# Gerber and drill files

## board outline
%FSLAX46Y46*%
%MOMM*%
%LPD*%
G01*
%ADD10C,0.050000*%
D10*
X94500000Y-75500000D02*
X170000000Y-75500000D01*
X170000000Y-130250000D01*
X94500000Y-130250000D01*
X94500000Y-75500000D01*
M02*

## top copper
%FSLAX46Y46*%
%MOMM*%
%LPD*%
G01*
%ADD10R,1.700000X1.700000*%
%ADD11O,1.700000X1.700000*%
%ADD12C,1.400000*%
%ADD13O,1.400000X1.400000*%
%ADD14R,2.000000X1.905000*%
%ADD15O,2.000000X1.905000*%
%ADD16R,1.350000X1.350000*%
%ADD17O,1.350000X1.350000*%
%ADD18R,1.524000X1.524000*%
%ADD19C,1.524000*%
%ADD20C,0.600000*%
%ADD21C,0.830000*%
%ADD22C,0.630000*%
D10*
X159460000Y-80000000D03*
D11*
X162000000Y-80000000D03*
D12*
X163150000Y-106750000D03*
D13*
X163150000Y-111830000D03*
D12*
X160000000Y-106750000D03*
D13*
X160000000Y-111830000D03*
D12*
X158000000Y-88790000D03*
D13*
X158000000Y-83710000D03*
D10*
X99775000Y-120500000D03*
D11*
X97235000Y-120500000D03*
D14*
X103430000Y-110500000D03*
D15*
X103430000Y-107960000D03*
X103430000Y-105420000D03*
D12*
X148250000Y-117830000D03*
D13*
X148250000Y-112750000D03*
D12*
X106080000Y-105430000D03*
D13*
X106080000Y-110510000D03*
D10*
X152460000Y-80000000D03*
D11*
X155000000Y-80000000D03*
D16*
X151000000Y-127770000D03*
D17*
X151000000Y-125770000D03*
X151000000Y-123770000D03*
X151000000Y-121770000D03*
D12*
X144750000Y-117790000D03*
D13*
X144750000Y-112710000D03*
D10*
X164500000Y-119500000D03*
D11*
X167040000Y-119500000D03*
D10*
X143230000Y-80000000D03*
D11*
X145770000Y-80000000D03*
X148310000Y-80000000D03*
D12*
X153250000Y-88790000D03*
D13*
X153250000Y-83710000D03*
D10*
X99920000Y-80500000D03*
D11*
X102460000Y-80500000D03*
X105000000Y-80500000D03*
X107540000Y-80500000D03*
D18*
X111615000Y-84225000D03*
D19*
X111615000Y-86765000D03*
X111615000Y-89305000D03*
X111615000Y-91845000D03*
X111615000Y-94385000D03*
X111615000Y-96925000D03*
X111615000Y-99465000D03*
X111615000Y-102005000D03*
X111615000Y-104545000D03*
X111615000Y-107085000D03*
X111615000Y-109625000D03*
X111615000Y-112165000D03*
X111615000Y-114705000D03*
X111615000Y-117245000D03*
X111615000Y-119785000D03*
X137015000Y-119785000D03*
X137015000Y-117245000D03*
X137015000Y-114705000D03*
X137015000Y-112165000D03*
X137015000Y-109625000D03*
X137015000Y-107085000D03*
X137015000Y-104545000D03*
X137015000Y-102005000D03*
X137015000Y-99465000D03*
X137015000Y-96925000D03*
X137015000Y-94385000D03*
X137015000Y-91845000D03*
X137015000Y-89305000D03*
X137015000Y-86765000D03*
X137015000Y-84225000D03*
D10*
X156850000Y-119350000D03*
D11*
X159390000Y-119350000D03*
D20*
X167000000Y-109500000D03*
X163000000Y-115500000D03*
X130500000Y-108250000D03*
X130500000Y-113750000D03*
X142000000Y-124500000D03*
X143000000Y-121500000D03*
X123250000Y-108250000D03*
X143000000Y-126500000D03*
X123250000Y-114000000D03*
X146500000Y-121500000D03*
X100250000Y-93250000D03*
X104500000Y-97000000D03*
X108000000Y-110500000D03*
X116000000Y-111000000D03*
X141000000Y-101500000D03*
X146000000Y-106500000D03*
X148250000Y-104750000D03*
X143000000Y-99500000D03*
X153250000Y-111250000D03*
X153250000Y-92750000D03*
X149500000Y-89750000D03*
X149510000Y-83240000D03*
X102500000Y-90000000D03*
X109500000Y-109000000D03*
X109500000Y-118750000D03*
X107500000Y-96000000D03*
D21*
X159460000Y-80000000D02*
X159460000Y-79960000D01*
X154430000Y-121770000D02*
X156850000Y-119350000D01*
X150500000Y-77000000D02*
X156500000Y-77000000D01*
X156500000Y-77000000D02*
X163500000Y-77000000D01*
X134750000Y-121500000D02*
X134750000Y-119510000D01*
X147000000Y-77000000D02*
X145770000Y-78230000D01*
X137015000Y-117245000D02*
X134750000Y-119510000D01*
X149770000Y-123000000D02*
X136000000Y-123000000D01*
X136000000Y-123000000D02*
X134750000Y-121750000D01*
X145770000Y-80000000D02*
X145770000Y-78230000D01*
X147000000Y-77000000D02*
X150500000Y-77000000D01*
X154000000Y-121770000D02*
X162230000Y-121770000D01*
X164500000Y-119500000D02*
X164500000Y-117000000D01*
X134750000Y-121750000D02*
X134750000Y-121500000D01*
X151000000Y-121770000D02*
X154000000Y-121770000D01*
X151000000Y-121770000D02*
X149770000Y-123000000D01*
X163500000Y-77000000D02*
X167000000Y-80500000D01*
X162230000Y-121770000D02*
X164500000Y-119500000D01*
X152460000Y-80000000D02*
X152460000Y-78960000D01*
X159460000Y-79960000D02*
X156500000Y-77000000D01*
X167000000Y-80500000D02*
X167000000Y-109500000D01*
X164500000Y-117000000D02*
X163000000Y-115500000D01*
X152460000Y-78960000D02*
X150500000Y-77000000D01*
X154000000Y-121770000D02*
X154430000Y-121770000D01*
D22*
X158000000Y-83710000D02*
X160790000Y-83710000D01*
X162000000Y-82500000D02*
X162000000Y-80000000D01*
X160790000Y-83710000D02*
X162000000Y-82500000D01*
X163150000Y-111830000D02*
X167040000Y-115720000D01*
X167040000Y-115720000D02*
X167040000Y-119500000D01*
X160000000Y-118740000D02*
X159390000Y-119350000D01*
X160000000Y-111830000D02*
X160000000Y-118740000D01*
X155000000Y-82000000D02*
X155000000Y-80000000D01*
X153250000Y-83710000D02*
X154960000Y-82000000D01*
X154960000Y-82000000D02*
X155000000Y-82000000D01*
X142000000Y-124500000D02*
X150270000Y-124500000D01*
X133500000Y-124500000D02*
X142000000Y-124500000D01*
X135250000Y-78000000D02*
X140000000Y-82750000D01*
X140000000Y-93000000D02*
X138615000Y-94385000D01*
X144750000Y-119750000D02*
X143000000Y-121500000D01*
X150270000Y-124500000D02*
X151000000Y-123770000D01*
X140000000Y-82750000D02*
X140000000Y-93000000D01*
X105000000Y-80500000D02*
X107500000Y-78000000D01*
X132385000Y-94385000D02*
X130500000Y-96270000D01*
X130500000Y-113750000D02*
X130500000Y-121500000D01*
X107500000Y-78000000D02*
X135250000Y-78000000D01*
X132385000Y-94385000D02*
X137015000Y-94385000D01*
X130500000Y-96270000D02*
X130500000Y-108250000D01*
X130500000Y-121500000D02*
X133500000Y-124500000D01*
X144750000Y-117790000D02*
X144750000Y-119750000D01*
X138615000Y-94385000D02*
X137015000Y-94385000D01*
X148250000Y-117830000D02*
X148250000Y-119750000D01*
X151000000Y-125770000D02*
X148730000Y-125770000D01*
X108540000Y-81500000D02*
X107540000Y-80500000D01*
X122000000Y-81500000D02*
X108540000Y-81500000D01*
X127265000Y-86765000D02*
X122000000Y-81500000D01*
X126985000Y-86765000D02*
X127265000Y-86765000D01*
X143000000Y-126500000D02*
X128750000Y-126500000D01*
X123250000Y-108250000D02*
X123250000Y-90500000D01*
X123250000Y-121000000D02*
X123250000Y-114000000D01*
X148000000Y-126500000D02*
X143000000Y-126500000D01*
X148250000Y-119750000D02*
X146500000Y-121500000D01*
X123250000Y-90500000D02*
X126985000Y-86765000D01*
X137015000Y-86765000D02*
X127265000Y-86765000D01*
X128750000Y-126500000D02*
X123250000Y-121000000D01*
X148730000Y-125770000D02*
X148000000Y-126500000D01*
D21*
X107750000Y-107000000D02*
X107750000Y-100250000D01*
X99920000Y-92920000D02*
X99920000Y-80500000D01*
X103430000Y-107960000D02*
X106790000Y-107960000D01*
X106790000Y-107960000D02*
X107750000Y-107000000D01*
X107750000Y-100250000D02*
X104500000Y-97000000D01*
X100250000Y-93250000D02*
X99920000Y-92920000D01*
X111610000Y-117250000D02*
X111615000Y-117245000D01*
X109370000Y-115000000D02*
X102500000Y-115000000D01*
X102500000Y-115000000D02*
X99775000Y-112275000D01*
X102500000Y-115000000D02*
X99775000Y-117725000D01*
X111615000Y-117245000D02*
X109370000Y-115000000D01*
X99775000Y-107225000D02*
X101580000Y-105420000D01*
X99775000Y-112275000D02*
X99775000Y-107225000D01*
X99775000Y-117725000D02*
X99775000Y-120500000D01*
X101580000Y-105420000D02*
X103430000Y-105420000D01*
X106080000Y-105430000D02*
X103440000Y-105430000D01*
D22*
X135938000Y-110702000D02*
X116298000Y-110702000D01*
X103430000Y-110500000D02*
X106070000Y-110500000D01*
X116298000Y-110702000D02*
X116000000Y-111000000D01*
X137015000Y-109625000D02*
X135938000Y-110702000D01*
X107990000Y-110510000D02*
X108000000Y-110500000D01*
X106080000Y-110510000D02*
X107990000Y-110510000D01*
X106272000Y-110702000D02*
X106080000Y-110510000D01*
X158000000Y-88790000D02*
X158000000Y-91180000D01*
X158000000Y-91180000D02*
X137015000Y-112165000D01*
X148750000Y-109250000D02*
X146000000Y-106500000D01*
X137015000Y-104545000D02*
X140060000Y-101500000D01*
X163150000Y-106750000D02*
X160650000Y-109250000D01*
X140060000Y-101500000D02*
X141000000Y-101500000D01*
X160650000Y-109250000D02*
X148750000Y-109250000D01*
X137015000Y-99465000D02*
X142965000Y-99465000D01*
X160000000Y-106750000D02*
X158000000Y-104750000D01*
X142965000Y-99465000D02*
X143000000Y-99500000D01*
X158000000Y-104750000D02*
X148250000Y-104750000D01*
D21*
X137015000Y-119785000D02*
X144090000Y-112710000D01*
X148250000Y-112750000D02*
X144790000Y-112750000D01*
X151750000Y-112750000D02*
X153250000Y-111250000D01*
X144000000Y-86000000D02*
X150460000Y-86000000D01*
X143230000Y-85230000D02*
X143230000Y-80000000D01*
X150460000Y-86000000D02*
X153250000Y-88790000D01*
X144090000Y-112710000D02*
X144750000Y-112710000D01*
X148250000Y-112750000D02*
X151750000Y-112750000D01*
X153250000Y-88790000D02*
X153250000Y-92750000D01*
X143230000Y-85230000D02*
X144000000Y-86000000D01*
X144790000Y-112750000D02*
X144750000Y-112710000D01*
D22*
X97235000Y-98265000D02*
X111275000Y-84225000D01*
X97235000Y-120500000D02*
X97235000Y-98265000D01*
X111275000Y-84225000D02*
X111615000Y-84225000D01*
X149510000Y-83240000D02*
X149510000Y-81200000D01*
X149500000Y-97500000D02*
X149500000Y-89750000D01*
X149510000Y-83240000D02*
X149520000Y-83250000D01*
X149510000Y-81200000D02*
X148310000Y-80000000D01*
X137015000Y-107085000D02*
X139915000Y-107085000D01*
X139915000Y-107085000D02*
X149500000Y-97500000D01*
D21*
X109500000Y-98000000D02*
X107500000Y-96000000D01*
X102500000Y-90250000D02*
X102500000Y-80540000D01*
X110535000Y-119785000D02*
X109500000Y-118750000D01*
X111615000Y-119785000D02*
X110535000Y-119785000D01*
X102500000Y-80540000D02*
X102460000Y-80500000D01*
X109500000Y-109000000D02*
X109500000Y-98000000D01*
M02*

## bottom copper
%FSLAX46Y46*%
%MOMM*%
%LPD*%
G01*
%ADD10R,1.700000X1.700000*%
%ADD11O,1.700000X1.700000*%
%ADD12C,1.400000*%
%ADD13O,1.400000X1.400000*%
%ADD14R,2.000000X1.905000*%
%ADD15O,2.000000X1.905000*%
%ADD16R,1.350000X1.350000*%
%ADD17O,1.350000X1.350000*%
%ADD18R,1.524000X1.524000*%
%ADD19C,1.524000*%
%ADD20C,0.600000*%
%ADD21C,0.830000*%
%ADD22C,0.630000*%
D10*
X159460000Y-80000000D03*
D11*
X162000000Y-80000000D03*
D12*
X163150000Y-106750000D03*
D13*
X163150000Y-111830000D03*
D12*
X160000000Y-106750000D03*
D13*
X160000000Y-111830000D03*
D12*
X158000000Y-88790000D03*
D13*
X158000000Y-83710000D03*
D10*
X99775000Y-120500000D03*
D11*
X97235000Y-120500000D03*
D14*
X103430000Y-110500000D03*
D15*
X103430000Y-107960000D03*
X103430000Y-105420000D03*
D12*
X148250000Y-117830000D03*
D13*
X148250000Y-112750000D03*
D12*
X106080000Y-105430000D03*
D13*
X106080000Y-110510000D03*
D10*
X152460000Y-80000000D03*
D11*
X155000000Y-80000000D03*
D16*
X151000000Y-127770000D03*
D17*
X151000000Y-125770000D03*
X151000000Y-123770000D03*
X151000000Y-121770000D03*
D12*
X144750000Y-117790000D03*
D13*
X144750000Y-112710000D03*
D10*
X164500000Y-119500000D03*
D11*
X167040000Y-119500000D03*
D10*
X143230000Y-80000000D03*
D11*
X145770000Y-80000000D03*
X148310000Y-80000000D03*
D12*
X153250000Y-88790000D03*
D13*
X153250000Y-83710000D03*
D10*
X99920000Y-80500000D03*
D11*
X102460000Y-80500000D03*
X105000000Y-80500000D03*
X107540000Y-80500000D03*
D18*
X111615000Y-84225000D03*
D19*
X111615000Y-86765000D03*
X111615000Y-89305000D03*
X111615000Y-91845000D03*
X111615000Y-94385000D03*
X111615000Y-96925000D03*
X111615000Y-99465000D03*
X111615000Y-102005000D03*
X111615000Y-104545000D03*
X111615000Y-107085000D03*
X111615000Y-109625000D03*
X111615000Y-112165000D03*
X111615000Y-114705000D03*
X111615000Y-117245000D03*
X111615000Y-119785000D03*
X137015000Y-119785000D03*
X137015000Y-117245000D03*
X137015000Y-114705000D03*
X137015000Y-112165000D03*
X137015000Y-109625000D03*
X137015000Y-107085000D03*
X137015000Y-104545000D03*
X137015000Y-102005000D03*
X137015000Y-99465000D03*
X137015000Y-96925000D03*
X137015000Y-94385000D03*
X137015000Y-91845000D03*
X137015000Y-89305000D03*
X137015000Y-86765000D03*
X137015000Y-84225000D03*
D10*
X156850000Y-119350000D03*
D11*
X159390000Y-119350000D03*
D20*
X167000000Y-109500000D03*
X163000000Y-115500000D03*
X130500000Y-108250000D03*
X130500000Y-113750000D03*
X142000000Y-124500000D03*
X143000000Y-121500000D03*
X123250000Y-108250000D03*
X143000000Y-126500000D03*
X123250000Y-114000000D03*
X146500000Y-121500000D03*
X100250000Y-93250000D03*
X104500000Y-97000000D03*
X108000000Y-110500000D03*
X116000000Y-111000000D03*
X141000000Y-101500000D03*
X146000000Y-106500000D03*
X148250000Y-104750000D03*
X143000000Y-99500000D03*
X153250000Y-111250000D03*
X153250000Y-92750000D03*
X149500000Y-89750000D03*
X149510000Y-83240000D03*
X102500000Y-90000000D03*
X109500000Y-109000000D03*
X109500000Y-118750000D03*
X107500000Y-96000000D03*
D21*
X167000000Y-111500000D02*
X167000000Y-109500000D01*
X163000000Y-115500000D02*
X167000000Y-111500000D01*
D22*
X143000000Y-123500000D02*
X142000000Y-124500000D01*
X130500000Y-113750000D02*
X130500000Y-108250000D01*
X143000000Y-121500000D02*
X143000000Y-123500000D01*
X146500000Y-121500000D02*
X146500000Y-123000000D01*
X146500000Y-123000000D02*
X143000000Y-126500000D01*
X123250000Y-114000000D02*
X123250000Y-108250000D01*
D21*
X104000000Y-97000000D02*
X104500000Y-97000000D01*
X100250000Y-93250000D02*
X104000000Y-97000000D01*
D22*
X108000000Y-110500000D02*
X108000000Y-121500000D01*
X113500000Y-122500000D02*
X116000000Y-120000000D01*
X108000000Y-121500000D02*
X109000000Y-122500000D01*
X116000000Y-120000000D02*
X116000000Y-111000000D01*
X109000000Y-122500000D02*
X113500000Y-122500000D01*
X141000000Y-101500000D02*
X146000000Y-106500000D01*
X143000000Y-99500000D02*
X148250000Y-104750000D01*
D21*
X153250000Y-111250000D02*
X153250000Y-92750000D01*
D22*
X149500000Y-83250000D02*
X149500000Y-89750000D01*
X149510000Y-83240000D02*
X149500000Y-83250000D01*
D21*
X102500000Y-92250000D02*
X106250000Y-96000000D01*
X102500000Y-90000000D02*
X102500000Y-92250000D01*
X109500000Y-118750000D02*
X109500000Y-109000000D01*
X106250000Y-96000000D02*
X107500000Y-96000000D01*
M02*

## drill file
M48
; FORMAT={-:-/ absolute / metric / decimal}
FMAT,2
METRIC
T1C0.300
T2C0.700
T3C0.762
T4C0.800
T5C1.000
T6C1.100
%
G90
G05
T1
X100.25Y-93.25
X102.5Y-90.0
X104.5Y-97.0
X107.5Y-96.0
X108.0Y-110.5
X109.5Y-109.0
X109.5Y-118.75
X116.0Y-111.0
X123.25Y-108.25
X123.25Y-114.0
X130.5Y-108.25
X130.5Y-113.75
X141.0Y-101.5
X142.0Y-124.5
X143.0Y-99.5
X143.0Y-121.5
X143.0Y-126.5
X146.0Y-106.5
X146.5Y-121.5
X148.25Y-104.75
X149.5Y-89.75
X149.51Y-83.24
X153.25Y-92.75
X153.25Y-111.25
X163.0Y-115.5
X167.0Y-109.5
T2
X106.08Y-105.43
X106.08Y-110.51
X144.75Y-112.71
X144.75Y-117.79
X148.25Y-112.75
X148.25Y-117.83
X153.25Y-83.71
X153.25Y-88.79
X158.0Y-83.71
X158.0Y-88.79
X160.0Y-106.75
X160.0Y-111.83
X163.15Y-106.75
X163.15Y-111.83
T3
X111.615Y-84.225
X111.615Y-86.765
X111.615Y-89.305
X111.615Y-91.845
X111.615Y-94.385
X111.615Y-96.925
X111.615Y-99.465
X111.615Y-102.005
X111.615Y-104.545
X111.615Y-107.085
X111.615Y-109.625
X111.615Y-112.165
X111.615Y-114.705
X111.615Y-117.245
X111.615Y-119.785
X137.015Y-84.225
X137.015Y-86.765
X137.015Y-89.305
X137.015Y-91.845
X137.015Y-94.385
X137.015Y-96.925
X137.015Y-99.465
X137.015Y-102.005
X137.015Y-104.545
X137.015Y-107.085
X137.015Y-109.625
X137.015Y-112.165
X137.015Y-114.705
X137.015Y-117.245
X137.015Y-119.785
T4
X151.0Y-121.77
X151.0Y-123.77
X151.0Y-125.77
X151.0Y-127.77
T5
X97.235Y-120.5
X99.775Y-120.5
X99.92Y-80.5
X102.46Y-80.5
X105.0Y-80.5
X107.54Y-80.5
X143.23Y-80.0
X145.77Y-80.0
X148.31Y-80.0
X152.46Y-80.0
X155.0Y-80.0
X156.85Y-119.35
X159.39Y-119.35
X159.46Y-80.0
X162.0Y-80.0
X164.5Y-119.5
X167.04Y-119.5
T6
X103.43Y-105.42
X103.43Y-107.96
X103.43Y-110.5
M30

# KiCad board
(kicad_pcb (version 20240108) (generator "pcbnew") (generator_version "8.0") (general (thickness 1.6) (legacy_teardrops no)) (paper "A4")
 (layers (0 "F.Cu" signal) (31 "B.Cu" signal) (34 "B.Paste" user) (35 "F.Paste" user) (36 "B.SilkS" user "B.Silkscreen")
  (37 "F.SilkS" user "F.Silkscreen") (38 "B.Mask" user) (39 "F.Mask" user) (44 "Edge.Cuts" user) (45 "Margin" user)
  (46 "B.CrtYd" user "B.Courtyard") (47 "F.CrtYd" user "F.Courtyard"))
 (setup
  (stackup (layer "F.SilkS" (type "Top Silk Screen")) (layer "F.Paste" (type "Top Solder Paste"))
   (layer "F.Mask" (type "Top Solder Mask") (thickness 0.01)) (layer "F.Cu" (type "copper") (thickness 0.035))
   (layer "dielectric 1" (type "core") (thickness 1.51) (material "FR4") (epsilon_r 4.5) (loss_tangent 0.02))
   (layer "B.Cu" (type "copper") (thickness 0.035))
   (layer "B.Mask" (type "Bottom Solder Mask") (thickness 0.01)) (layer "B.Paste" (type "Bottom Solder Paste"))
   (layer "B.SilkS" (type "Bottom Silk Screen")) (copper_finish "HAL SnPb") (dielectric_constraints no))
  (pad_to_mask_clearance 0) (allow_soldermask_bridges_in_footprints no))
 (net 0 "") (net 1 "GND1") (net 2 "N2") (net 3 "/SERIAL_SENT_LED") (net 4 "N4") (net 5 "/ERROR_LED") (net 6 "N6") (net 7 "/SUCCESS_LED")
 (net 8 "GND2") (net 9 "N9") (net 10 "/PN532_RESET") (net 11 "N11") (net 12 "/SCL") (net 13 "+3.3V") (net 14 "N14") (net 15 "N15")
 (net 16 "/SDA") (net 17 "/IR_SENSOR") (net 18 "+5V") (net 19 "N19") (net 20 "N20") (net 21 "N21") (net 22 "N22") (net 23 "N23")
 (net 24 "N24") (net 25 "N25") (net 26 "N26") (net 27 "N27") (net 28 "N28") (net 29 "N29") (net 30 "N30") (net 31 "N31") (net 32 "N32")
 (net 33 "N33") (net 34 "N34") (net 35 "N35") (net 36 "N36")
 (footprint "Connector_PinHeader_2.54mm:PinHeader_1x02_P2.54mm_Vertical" (layer "F.Cu") (at 159.46 80 90)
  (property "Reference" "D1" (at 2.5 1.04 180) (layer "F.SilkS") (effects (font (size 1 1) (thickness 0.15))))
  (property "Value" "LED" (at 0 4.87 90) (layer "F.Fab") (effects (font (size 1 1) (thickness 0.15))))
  (pad "1" thru_hole rect (at 0 0 90) (size 1.7 1.7) (drill 1) (layers "*.Cu" "*.Mask") (remove_unused_layers no) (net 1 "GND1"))
  (pad "2" thru_hole oval (at 0 2.54 90) (size 1.7 1.7) (drill 1) (layers "*.Cu" "*.Mask") (remove_unused_layers no) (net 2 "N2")))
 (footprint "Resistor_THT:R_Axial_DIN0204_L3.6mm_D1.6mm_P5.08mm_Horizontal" (layer "F.Cu") (at 163.15 106.75 -90)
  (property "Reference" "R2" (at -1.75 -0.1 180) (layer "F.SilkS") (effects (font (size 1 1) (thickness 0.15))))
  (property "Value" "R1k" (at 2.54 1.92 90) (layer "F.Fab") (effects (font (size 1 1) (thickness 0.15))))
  (pad "1" thru_hole circle (at 0 0 270) (size 1.4 1.4) (drill 0.7) (layers "*.Cu" "*.Mask") (remove_unused_layers no)
   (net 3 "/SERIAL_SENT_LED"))
  (pad "2" thru_hole oval (at 5.08 0 270) (size 1.4 1.4) (drill 0.7) (layers "*.Cu" "*.Mask") (remove_unused_layers no) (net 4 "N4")))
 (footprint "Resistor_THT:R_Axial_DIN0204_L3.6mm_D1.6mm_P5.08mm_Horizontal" (layer "F.Cu") (at 160 106.75 -90)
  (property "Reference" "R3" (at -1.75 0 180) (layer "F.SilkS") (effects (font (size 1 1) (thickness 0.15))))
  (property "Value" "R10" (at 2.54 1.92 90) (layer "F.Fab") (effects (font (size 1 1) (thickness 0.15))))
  (pad "1" thru_hole circle (at 0 0 270) (size 1.4 1.4) (drill 0.7) (layers "*.Cu" "*.Mask") (remove_unused_layers no) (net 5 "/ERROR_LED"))
  (pad "2" thru_hole oval (at 5.08 0 270) (size 1.4 1.4) (drill 0.7) (layers "*.Cu" "*.Mask") (remove_unused_layers no) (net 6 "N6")))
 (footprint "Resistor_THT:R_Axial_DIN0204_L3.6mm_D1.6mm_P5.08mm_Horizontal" (layer "F.Cu") (at 158 88.79 90)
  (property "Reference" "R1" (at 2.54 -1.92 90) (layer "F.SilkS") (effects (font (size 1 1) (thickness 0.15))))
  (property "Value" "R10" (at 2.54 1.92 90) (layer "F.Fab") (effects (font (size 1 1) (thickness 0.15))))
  (pad "1" thru_hole circle (at 0 0 90) (size 1.4 1.4) (drill 0.7) (layers "*.Cu" "*.Mask") (remove_unused_layers no) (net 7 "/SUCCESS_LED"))
  (pad "2" thru_hole oval (at 5.08 0 90) (size 1.4 1.4) (drill 0.7) (layers "*.Cu" "*.Mask") (remove_unused_layers no) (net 2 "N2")))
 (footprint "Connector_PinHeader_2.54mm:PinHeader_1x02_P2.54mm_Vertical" (layer "F.Cu") (at 99.775 120.5 -90)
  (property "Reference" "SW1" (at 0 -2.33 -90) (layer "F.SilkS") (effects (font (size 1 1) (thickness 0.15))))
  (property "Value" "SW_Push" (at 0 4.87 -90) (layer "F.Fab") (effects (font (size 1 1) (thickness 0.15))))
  (pad "1" thru_hole rect (at 0 0 270) (size 1.7 1.7) (drill 1) (layers "*.Cu" "*.Mask") (remove_unused_layers no) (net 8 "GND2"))
  (pad "2" thru_hole oval (at 0 2.54 270) (size 1.7 1.7) (drill 1) (layers "*.Cu" "*.Mask") (remove_unused_layers no) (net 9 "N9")))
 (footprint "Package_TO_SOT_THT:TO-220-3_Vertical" (layer "F.Cu") (at 103.43 110.5 90)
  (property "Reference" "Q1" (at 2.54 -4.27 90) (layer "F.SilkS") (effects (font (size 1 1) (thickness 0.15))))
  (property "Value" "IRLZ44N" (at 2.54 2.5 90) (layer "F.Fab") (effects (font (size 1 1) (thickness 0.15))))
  (pad "1" thru_hole rect (at 0 0 90) (size 1.905 2) (drill 1.1) (layers "*.Cu" "*.Mask") (remove_unused_layers no) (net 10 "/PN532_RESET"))
  (pad "2" thru_hole oval (at 2.54 0 90) (size 1.905 2) (drill 1.1) (layers "*.Cu" "*.Mask") (remove_unused_layers no) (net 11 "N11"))
  (pad "3" thru_hole oval (at 5.08 0 90) (size 1.905 2) (drill 1.1) (layers "*.Cu" "*.Mask") (remove_unused_layers no) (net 8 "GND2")))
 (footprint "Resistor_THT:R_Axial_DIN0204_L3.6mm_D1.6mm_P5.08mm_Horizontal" (layer "F.Cu") (at 148.25 117.83 90)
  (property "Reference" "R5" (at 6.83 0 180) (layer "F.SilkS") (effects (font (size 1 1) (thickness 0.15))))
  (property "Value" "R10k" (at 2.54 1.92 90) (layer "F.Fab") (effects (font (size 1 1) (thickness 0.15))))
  (pad "1" thru_hole circle (at 0 0 90) (size 1.4 1.4) (drill 0.7) (layers "*.Cu" "*.Mask") (remove_unused_layers no) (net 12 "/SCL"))
  (pad "2" thru_hole oval (at 5.08 0 90) (size 1.4 1.4) (drill 0.7) (layers "*.Cu" "*.Mask") (remove_unused_layers no) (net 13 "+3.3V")))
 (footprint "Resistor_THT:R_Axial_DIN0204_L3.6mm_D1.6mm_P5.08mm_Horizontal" (layer "F.Cu") (at 106.08 105.43 -90)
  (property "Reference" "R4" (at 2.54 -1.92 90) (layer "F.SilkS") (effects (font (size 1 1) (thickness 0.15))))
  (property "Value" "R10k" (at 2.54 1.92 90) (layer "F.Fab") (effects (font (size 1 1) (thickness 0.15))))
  (pad "1" thru_hole circle (at 0 0 270) (size 1.4 1.4) (drill 0.7) (layers "*.Cu" "*.Mask") (remove_unused_layers no) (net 8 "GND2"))
  (pad "2" thru_hole oval (at 5.08 0 270) (size 1.4 1.4) (drill 0.7) (layers "*.Cu" "*.Mask") (remove_unused_layers no)
   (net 10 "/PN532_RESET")))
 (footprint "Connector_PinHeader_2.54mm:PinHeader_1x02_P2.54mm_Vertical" (layer "F.Cu") (at 152.46 80 90)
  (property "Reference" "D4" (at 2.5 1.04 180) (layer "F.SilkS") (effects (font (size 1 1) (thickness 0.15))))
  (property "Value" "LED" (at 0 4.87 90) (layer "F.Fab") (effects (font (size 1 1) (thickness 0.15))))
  (pad "1" thru_hole rect (at 0 0 90) (size 1.7 1.7) (drill 1) (layers "*.Cu" "*.Mask") (remove_unused_layers no) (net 1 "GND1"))
  (pad "2" thru_hole oval (at 0 2.54 90) (size 1.7 1.7) (drill 1) (layers "*.Cu" "*.Mask") (remove_unused_layers no) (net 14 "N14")))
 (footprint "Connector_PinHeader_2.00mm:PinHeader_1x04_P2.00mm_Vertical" (layer "F.Cu") (at 151 127.77 180)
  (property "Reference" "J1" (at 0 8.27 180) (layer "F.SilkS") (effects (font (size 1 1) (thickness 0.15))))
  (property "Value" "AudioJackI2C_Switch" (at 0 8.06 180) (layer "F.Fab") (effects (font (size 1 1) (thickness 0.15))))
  (pad "1" thru_hole rect (at 0 0 180) (size 1.35 1.35) (drill 0.8) (layers "*.Cu" "*.Mask") (remove_unused_layers no) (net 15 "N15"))
  (pad "2" thru_hole oval (at 0 2 180) (size 1.35 1.35) (drill 0.8) (layers "*.Cu" "*.Mask") (remove_unused_layers no) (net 12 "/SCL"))
  (pad "3" thru_hole oval (at 0 4 180) (size 1.35 1.35) (drill 0.8) (layers "*.Cu" "*.Mask") (remove_unused_layers no) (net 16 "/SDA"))
  (pad "4" thru_hole oval (at 0 6 180) (size 1.35 1.35) (drill 0.8) (layers "*.Cu" "*.Mask") (remove_unused_layers no) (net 1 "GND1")))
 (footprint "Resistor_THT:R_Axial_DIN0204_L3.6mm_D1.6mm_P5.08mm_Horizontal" (layer "F.Cu") (at 144.75 117.79 90)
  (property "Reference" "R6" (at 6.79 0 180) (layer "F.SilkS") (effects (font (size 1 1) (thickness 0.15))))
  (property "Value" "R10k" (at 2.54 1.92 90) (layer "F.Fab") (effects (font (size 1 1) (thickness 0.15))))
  (pad "1" thru_hole circle (at 0 0 90) (size 1.4 1.4) (drill 0.7) (layers "*.Cu" "*.Mask") (remove_unused_layers no) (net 16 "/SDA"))
  (pad "2" thru_hole oval (at 5.08 0 90) (size 1.4 1.4) (drill 0.7) (layers "*.Cu" "*.Mask") (remove_unused_layers no) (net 13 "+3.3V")))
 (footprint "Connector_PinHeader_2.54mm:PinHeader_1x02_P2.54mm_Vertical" (layer "F.Cu") (at 164.5 119.5 90)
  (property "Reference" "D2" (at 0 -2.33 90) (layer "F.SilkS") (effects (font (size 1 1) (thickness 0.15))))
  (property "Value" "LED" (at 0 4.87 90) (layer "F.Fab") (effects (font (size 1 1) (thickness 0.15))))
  (pad "1" thru_hole rect (at 0 0 90) (size 1.7 1.7) (drill 1) (layers "*.Cu" "*.Mask") (remove_unused_layers no) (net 1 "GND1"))
  (pad "2" thru_hole oval (at 0 2.54 90) (size 1.7 1.7) (drill 1) (layers "*.Cu" "*.Mask") (remove_unused_layers no) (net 4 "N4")))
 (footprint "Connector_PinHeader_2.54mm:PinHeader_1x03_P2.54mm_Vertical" (layer "F.Cu") (at 143.23 80 90)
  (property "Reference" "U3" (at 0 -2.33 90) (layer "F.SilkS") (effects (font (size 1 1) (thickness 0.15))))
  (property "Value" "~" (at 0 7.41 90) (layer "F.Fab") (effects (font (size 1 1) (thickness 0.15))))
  (pad "1" thru_hole rect (at 0 0 90) (size 1.7 1.7) (drill 1) (layers "*.Cu" "*.Mask") (remove_unused_layers no) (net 13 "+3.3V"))
  (pad "2" thru_hole oval (at 0 2.54 90) (size 1.7 1.7) (drill 1) (layers "*.Cu" "*.Mask") (remove_unused_layers no) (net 1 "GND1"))
  (pad "3" thru_hole oval (at 0 5.08 90) (size 1.7 1.7) (drill 1) (layers "*.Cu" "*.Mask") (remove_unused_layers no) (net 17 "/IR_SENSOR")))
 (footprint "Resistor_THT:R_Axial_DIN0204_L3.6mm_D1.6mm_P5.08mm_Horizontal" (layer "F.Cu") (at 153.25 88.79 90)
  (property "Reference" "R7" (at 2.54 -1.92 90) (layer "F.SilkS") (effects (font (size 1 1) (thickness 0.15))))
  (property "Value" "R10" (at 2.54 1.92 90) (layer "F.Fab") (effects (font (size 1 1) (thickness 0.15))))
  (pad "1" thru_hole circle (at 0 0 90) (size 1.4 1.4) (drill 0.7) (layers "*.Cu" "*.Mask") (remove_unused_layers no) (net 13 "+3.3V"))
  (pad "2" thru_hole oval (at 5.08 0 90) (size 1.4 1.4) (drill 0.7) (layers "*.Cu" "*.Mask") (remove_unused_layers no) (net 14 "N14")))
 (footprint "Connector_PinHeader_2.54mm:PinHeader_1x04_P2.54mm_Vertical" (layer "F.Cu") (at 99.92 80.5 90)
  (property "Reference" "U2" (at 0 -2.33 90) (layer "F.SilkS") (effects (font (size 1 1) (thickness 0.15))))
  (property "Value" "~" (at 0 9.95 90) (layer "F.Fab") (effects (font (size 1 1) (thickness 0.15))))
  (pad "1" thru_hole rect (at 0 0 90) (size 1.7 1.7) (drill 1) (layers "*.Cu" "*.Mask") (remove_unused_layers no) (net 11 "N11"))
  (pad "2" thru_hole oval (at 0 2.54 90) (size 1.7 1.7) (drill 1) (layers "*.Cu" "*.Mask") (remove_unused_layers no) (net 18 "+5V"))
  (pad "3" thru_hole oval (at 0 5.08 90) (size 1.7 1.7) (drill 1) (layers "*.Cu" "*.Mask") (remove_unused_layers no) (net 16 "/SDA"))
  (pad "4" thru_hole oval (at 0 7.62 90) (size 1.7 1.7) (drill 1) (layers "*.Cu" "*.Mask") (remove_unused_layers no) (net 12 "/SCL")))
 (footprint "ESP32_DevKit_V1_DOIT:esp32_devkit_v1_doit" (layer "F.Cu") (at 124.315 84.225)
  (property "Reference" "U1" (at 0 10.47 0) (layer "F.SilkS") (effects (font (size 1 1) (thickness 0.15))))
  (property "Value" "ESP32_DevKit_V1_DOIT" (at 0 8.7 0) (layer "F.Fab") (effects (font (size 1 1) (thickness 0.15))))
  (pad "1" thru_hole rect (at -12.7 0) (size 1.524 1.524) (drill 0.762) (layers "*.Cu" "*.Mask") (remove_unused_layers no) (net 9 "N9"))
  (pad "2" thru_hole circle (at -12.7 2.54) (size 1.524 1.524) (drill 0.762) (layers "*.Cu" "*.Mask") (remove_unused_layers no)
   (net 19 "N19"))
  (pad "3" thru_hole circle (at -12.7 5.08) (size 1.524 1.524) (drill 0.762) (layers "*.Cu" "*.Mask") (remove_unused_layers no)
   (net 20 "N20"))
  (pad "4" thru_hole circle (at -12.7 7.62) (size 1.524 1.524) (drill 0.762) (layers "*.Cu" "*.Mask") (remove_unused_layers no)
   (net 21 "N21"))
  (pad "5" thru_hole circle (at -12.7 10.16) (size 1.524 1.524) (drill 0.762) (layers "*.Cu" "*.Mask") (remove_unused_layers no)
   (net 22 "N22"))
  (pad "6" thru_hole circle (at -12.7 12.7) (size 1.524 1.524) (drill 0.762) (layers "*.Cu" "*.Mask") (remove_unused_layers no)
   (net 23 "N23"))
  (pad "7" thru_hole circle (at -12.7 15.24) (size 1.524 1.524) (drill 0.762) (layers "*.Cu" "*.Mask") (remove_unused_layers no)
   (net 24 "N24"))
  (pad "8" thru_hole circle (at -12.7 17.78) (size 1.524 1.524) (drill 0.762) (layers "*.Cu" "*.Mask") (remove_unused_layers no)
   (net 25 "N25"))
  (pad "9" thru_hole circle (at -12.7 20.32) (size 1.524 1.524) (drill 0.762) (layers "*.Cu" "*.Mask") (remove_unused_layers no)
   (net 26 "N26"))
  (pad "10" thru_hole circle (at -12.7 22.86) (size 1.524 1.524) (drill 0.762) (layers "*.Cu" "*.Mask") (remove_unused_layers no)
   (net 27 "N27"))
  (pad "11" thru_hole circle (at -12.7 25.4) (size 1.524 1.524) (drill 0.762) (layers "*.Cu" "*.Mask") (remove_unused_layers no)
   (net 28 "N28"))
  (pad "12" thru_hole circle (at -12.7 27.94) (size 1.524 1.524) (drill 0.762) (layers "*.Cu" "*.Mask") (remove_unused_layers no)
   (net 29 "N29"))
  (pad "13" thru_hole circle (at -12.7 30.48) (size 1.524 1.524) (drill 0.762) (layers "*.Cu" "*.Mask") (remove_unused_layers no)
   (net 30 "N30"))
  (pad "14" thru_hole circle (at -12.7 33.02) (size 1.524 1.524) (drill 0.762) (layers "*.Cu" "*.Mask") (remove_unused_layers no)
   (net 8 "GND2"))
  (pad "15" thru_hole circle (at -12.7 35.56) (size 1.524 1.524) (drill 0.762) (layers "*.Cu" "*.Mask") (remove_unused_layers no)
   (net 18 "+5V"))
  (pad "16" thru_hole circle (at 12.7 35.56) (size 1.524 1.524) (drill 0.762) (layers "*.Cu" "*.Mask") (remove_unused_layers no)
   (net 13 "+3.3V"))
  (pad "17" thru_hole circle (at 12.7 33.02) (size 1.524 1.524) (drill 0.762) (layers "*.Cu" "*.Mask") (remove_unused_layers no)
   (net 1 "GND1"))
  (pad "18" thru_hole circle (at 12.7 30.48) (size 1.524 1.524) (drill 0.762) (layers "*.Cu" "*.Mask") (remove_unused_layers no)
   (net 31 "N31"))
  (pad "19" thru_hole circle (at 12.7 27.94) (size 1.524 1.524) (drill 0.762) (layers "*.Cu" "*.Mask") (remove_unused_layers no)
   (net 7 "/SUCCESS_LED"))
  (pad "20" thru_hole circle (at 12.7 25.4) (size 1.524 1.524) (drill 0.762) (layers "*.Cu" "*.Mask") (remove_unused_layers no)
   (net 10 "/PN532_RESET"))
  (pad "21" thru_hole circle (at 12.7 22.86) (size 1.524 1.524) (drill 0.762) (layers "*.Cu" "*.Mask") (remove_unused_layers no)
   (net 17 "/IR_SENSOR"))
  (pad "22" thru_hole circle (at 12.7 20.32) (size 1.524 1.524) (drill 0.762) (layers "*.Cu" "*.Mask") (remove_unused_layers no)
   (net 3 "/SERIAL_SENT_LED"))
  (pad "23" thru_hole circle (at 12.7 17.78) (size 1.524 1.524) (drill 0.762) (layers "*.Cu" "*.Mask") (remove_unused_layers no)
   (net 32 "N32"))
  (pad "24" thru_hole circle (at 12.7 15.24) (size 1.524 1.524) (drill 0.762) (layers "*.Cu" "*.Mask") (remove_unused_layers no)
   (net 5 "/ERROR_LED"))
  (pad "25" thru_hole circle (at 12.7 12.7) (size 1.524 1.524) (drill 0.762) (layers "*.Cu" "*.Mask") (remove_unused_layers no)
   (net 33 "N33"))
  (pad "26" thru_hole circle (at 12.7 10.16) (size 1.524 1.524) (drill 0.762) (layers "*.Cu" "*.Mask") (remove_unused_layers no)
   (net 16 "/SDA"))
  (pad "27" thru_hole circle (at 12.7 7.62) (size 1.524 1.524) (drill 0.762) (layers "*.Cu" "*.Mask") (remove_unused_layers no)
   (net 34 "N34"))
  (pad "28" thru_hole circle (at 12.7 5.08) (size 1.524 1.524) (drill 0.762) (layers "*.Cu" "*.Mask") (remove_unused_layers no)
   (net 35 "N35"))
  (pad "29" thru_hole circle (at 12.7 2.54) (size 1.524 1.524) (drill 0.762) (layers "*.Cu" "*.Mask") (remove_unused_layers no)
   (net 12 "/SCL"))
  (pad "30" thru_hole circle (at 12.7 0) (size 1.524 1.524) (drill 0.762) (layers "*.Cu" "*.Mask") (remove_unused_layers no) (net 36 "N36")))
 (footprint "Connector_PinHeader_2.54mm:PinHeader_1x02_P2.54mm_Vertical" (layer "F.Cu") (at 156.85 119.35 90)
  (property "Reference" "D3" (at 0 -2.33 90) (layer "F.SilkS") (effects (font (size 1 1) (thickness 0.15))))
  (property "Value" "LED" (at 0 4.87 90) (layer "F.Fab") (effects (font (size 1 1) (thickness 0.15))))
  (pad "1" thru_hole rect (at 0 0 90) (size 1.7 1.7) (drill 1) (layers "*.Cu" "*.Mask") (remove_unused_layers no) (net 1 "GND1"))
  (pad "2" thru_hole oval (at 0 2.54 90) (size 1.7 1.7) (drill 1) (layers "*.Cu" "*.Mask") (remove_unused_layers no) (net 6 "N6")))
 (gr_rect (start 94.5 75.5) (end 170 130.25) (locked yes) (stroke (width 0.05) (type default)) (fill none) (layer "Edge.Cuts"))
 (segment (start 159.46 80) (end 159.46 79.96) (width 0.83) (layer "F.Cu") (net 1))
 (segment (start 154.43 121.77) (end 156.85 119.35) (width 0.83) (layer "F.Cu") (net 1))
 (segment (start 150.5 77) (end 156.5 77) (width 0.83) (layer "F.Cu") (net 1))
 (segment (start 156.5 77) (end 163.5 77) (width 0.83) (layer "F.Cu") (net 1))
 (segment (start 134.75 121.5) (end 134.75 119.51) (width 0.83) (layer "F.Cu") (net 1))
 (segment (start 147 77) (end 145.77 78.23) (width 0.83) (layer "F.Cu") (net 1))
 (segment (start 137.015 117.245) (end 134.75 119.51) (width 0.83) (layer "F.Cu") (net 1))
 (segment (start 149.77 123) (end 136 123) (width 0.83) (layer "F.Cu") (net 1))
 (segment (start 136 123) (end 134.75 121.75) (width 0.83) (layer "F.Cu") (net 1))
 (segment (start 145.77 80) (end 145.77 78.23) (width 0.83) (layer "F.Cu") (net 1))
 (segment (start 147 77) (end 150.5 77) (width 0.83) (layer "F.Cu") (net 1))
 (segment (start 154 121.77) (end 162.23 121.77) (width 0.83) (layer "F.Cu") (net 1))
 (segment (start 164.5 119.5) (end 164.5 117) (width 0.83) (layer "F.Cu") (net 1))
 (segment (start 134.75 121.75) (end 134.75 121.5) (width 0.83) (layer "F.Cu") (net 1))
 (segment (start 151 121.77) (end 154 121.77) (width 0.83) (layer "F.Cu") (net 1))
 (segment (start 151 121.77) (end 149.77 123) (width 0.83) (layer "F.Cu") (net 1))
 (segment (start 163.5 77) (end 167 80.5) (width 0.83) (layer "F.Cu") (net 1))
 (segment (start 162.23 121.77) (end 164.5 119.5) (width 0.83) (layer "F.Cu") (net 1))
 (segment (start 152.46 80) (end 152.46 78.96) (width 0.83) (layer "F.Cu") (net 1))
 (segment (start 159.46 79.96) (end 156.5 77) (width 0.83) (layer "F.Cu") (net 1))
 (segment (start 167 80.5) (end 167 109.5) (width 0.83) (layer "F.Cu") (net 1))
 (segment (start 164.5 117) (end 163 115.5) (width 0.83) (layer "F.Cu") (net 1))
 (segment (start 152.46 78.96) (end 150.5 77) (width 0.83) (layer "F.Cu") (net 1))
 (segment (start 154 121.77) (end 154.43 121.77) (width 0.83) (layer "F.Cu") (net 1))
 (via (at 167 109.5) (size 0.6) (drill 0.3) (layers "F.Cu" "B.Cu") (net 1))
 (via (at 163 115.5) (size 0.6) (drill 0.3) (layers "F.Cu" "B.Cu") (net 1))
 (segment (start 167 111.5) (end 167 109.5) (width 0.83) (layer "B.Cu") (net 1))
 (segment (start 163 115.5) (end 167 111.5) (width 0.83) (layer "B.Cu") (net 1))
 (segment (start 158 83.71) (end 160.79 83.71) (width 0.63) (layer "F.Cu") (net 2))
 (segment (start 162 82.5) (end 162 80) (width 0.63) (layer "F.Cu") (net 2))
 (segment (start 160.79 83.71) (end 162 82.5) (width 0.63) (layer "F.Cu") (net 2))
 (segment (start 163.15 111.83) (end 167.04 115.72) (width 0.63) (layer "F.Cu") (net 4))
 (segment (start 167.04 115.72) (end 167.04 119.5) (width 0.63) (layer "F.Cu") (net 4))
 (segment (start 160 118.74) (end 159.39 119.35) (width 0.63) (layer "F.Cu") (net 6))
 (segment (start 160 111.83) (end 160 118.74) (width 0.63) (layer "F.Cu") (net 6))
 (segment (start 155 82) (end 155 80) (width 0.63) (layer "F.Cu") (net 14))
 (segment (start 153.25 83.71) (end 154.96 82) (width 0.63) (layer "F.Cu") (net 14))
 (segment (start 154.96 82) (end 155 82) (width 0.63) (layer "F.Cu") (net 14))
 (segment (start 142 124.5) (end 150.27 124.5) (width 0.63) (layer "F.Cu") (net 16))
 (segment (start 133.5 124.5) (end 142 124.5) (width 0.63) (layer "F.Cu") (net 16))
 (segment (start 135.25 78) (end 140 82.75) (width 0.63) (layer "F.Cu") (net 16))
 (segment (start 140 93) (end 138.615 94.385) (width 0.63) (layer "F.Cu") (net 16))
 (segment (start 144.75 119.75) (end 143 121.5) (width 0.63) (layer "F.Cu") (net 16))
 (segment (start 150.27 124.5) (end 151 123.77) (width 0.63) (layer "F.Cu") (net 16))
 (segment (start 140 82.75) (end 140 93) (width 0.63) (layer "F.Cu") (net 16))
 (segment (start 105 80.5) (end 107.5 78) (width 0.63) (layer "F.Cu") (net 16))
 (segment (start 132.385 94.385) (end 130.5 96.27) (width 0.63) (layer "F.Cu") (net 16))
 (segment (start 130.5 113.75) (end 130.5 121.5) (width 0.63) (layer "F.Cu") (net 16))
 (segment (start 107.5 78) (end 135.25 78) (width 0.63) (layer "F.Cu") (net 16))
 (segment (start 132.385 94.385) (end 137.015 94.385) (width 0.63) (layer "F.Cu") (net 16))
 (segment (start 130.5 96.27) (end 130.5 108.25) (width 0.63) (layer "F.Cu") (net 16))
 (segment (start 130.5 121.5) (end 133.5 124.5) (width 0.63) (layer "F.Cu") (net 16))
 (segment (start 144.75 117.79) (end 144.75 119.75) (width 0.63) (layer "F.Cu") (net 16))
 (segment (start 138.615 94.385) (end 137.015 94.385) (width 0.63) (layer "F.Cu") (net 16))
 (via (at 130.5 108.25) (size 0.6) (drill 0.3) (layers "F.Cu" "B.Cu") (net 16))
 (via (at 130.5 113.75) (size 0.6) (drill 0.3) (layers "F.Cu" "B.Cu") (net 16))
 (via (at 142 124.5) (size 0.6) (drill 0.3) (layers "F.Cu" "B.Cu") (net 16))
 (via (at 143 121.5) (size 0.6) (drill 0.3) (layers "F.Cu" "B.Cu") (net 16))
 (segment (start 143 123.5) (end 142 124.5) (width 0.63) (layer "B.Cu") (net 16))
 (segment (start 130.5 113.75) (end 130.5 108.25) (width 0.63) (layer "B.Cu") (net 16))
 (segment (start 143 121.5) (end 143 123.5) (width 0.63) (layer "B.Cu") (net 16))
 (segment (start 148.25 117.83) (end 148.25 119.75) (width 0.63) (layer "F.Cu") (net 12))
 (segment (start 151 125.77) (end 148.73 125.77) (width 0.63) (layer "F.Cu") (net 12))
 (segment (start 108.54 81.5) (end 107.54 80.5) (width 0.63) (layer "F.Cu") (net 12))
 (segment (start 122 81.5) (end 108.54 81.5) (width 0.63) (layer "F.Cu") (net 12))
 (segment (start 127.265 86.765) (end 122 81.5) (width 0.63) (layer "F.Cu") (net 12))
 (segment (start 126.985 86.765) (end 127.265 86.765) (width 0.63) (layer "F.Cu") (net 12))
 (segment (start 143 126.5) (end 128.75 126.5) (width 0.63) (layer "F.Cu") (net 12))
 (segment (start 123.25 108.25) (end 123.25 90.5) (width 0.63) (layer "F.Cu") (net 12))
 (segment (start 123.25 121) (end 123.25 114) (width 0.63) (layer "F.Cu") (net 12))
 (segment (start 148 126.5) (end 143 126.5) (width 0.63) (layer "F.Cu") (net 12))
 (segment (start 148.25 119.75) (end 146.5 121.5) (width 0.63) (layer "F.Cu") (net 12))
 (segment (start 123.25 90.5) (end 126.985 86.765) (width 0.63) (layer "F.Cu") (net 12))
 (segment (start 137.015 86.765) (end 127.265 86.765) (width 0.63) (layer "F.Cu") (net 12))
 (segment (start 128.75 126.5) (end 123.25 121) (width 0.63) (layer "F.Cu") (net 12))
 (segment (start 148.73 125.77) (end 148 126.5) (width 0.63) (layer "F.Cu") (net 12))
 (via (at 123.25 108.25) (size 0.6) (drill 0.3) (layers "F.Cu" "B.Cu") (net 12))
 (via (at 143 126.5) (size 0.6) (drill 0.3) (layers "F.Cu" "B.Cu") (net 12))
 (via (at 123.25 114) (size 0.6) (drill 0.3) (layers "F.Cu" "B.Cu") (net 12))
 (via (at 146.5 121.5) (size 0.6) (drill 0.3) (layers "F.Cu" "B.Cu") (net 12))
 (segment (start 146.5 121.5) (end 146.5 123) (width 0.63) (layer "B.Cu") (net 12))
 (segment (start 146.5 123) (end 143 126.5) (width 0.63) (layer "B.Cu") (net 12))
 (segment (start 123.25 114) (end 123.25 108.25) (width 0.63) (layer "B.Cu") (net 12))
 (segment (start 107.75 107) (end 107.75 100.25) (width 0.83) (layer "F.Cu") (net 11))
 (segment (start 99.92 92.92) (end 99.92 80.5) (width 0.83) (layer "F.Cu") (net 11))
 (segment (start 103.43 107.96) (end 106.79 107.96) (width 0.83) (layer "F.Cu") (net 11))
 (segment (start 106.79 107.96) (end 107.75 107) (width 0.83) (layer "F.Cu") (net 11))
 (segment (start 107.75 100.25) (end 104.5 97) (width 0.83) (layer "F.Cu") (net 11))
 (segment (start 100.25 93.25) (end 99.92 92.92) (width 0.83) (layer "F.Cu") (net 11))
 (via (at 100.25 93.25) (size 0.6) (drill 0.3) (layers "F.Cu" "B.Cu") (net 11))
 (via (at 104.5 97) (size 0.6) (drill 0.3) (layers "F.Cu" "B.Cu") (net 11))
 (segment (start 104 97) (end 104.5 97) (width 0.83) (layer "B.Cu") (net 11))
 (segment (start 100.25 93.25) (end 104 97) (width 0.83) (layer "B.Cu") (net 11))
 (segment (start 111.61 117.25) (end 111.615 117.245) (width 0.83) (layer "F.Cu") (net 8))
 (segment (start 109.37 115) (end 102.5 115) (width 0.83) (layer "F.Cu") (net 8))
 (segment (start 102.5 115) (end 99.775 112.275) (width 0.83) (layer "F.Cu") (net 8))
 (segment (start 102.5 115) (end 99.775 117.725) (width 0.83) (layer "F.Cu") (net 8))
 (segment (start 111.615 117.245) (end 109.37 115) (width 0.83) (layer "F.Cu") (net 8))
 (segment (start 99.775 107.225) (end 101.58 105.42) (width 0.83) (layer "F.Cu") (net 8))
 (segment (start 99.775 112.275) (end 99.775 107.225) (width 0.83) (layer "F.Cu") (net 8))
 (segment (start 99.775 117.725) (end 99.775 120.5) (width 0.83) (layer "F.Cu") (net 8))
 (segment (start 101.58 105.42) (end 103.43 105.42) (width 0.83) (layer "F.Cu") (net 8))
 (segment (start 106.08 105.43) (end 103.44 105.43) (width 0.83) (layer "F.Cu") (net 8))
 (segment (start 135.938 110.702) (end 116.298 110.702) (width 0.63) (layer "F.Cu") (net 10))
 (segment (start 103.43 110.5) (end 106.07 110.5) (width 0.63) (layer "F.Cu") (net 10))
 (segment (start 116.298 110.702) (end 116 111) (width 0.63) (layer "F.Cu") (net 10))
 (segment (start 137.015 109.625) (end 135.938 110.702) (width 0.63) (layer "F.Cu") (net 10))
 (segment (start 107.99 110.51) (end 108 110.5) (width 0.63) (layer "F.Cu") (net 10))
 (segment (start 106.08 110.51) (end 107.99 110.51) (width 0.63) (layer "F.Cu") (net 10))
 (segment (start 106.272 110.702) (end 106.08 110.51) (width 0.63) (layer "F.Cu") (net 10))
 (via (at 108 110.5) (size 0.6) (drill 0.3) (layers "F.Cu" "B.Cu") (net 10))
 (via (at 116 111) (size 0.6) (drill 0.3) (layers "F.Cu" "B.Cu") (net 10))
 (segment (start 108 110.5) (end 108 121.5) (width 0.63) (layer "B.Cu") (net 10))
 (segment (start 113.5 122.5) (end 116 120) (width 0.63) (layer "B.Cu") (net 10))
 (segment (start 108 121.5) (end 109 122.5) (width 0.63) (layer "B.Cu") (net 10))
 (segment (start 116 120) (end 116 111) (width 0.63) (layer "B.Cu") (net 10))
 (segment (start 109 122.5) (end 113.5 122.5) (width 0.63) (layer "B.Cu") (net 10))
 (segment (start 158 88.79) (end 158 91.18) (width 0.63) (layer "F.Cu") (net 7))
 (segment (start 158 91.18) (end 137.015 112.165) (width 0.63) (layer "F.Cu") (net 7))
 (segment (start 148.75 109.25) (end 146 106.5) (width 0.63) (layer "F.Cu") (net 3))
 (segment (start 137.015 104.545) (end 140.06 101.5) (width 0.63) (layer "F.Cu") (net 3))
 (segment (start 163.15 106.75) (end 160.65 109.25) (width 0.63) (layer "F.Cu") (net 3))
 (segment (start 140.06 101.5) (end 141 101.5) (width 0.63) (layer "F.Cu") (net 3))
 (segment (start 160.65 109.25) (end 148.75 109.25) (width 0.63) (layer "F.Cu") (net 3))
 (via (at 141 101.5) (size 0.6) (drill 0.3) (layers "F.Cu" "B.Cu") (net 3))
 (via (at 146 106.5) (size 0.6) (drill 0.3) (layers "F.Cu" "B.Cu") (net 3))
 (segment (start 141 101.5) (end 146 106.5) (width 0.63) (layer "B.Cu") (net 3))
 (segment (start 137.015 99.465) (end 142.965 99.465) (width 0.63) (layer "F.Cu") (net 5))
 (segment (start 160 106.75) (end 158 104.75) (width 0.63) (layer "F.Cu") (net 5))
 (segment (start 142.965 99.465) (end 143 99.5) (width 0.63) (layer "F.Cu") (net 5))
 (segment (start 158 104.75) (end 148.25 104.75) (width 0.63) (layer "F.Cu") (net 5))
 (via (at 148.25 104.75) (size 0.6) (drill 0.3) (layers "F.Cu" "B.Cu") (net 5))
 (via (at 143 99.5) (size 0.6) (drill 0.3) (layers "F.Cu" "B.Cu") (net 5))
 (segment (start 143 99.5) (end 148.25 104.75) (width 0.63) (layer "B.Cu") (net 5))
 (segment (start 137.015 119.785) (end 144.09 112.71) (width 0.83) (layer "F.Cu") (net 13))
 (segment (start 148.25 112.75) (end 144.79 112.75) (width 0.83) (layer "F.Cu") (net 13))
 (segment (start 151.75 112.75) (end 153.25 111.25) (width 0.83) (layer "F.Cu") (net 13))
 (segment (start 144 86) (end 150.46 86) (width 0.83) (layer "F.Cu") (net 13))
 (segment (start 143.23 85.23) (end 143.23 80) (width 0.83) (layer "F.Cu") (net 13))
 (segment (start 150.46 86) (end 153.25 88.79) (width 0.83) (layer "F.Cu") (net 13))
 (segment (start 144.09 112.71) (end 144.75 112.71) (width 0.83) (layer "F.Cu") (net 13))
 (segment (start 148.25 112.75) (end 151.75 112.75) (width 0.83) (layer "F.Cu") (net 13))
 (segment (start 153.25 88.79) (end 153.25 92.75) (width 0.83) (layer "F.Cu") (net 13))
 (segment (start 143.23 85.23) (end 144 86) (width 0.83) (layer "F.Cu") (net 13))
 (segment (start 144.79 112.75) (end 144.75 112.71) (width 0.83) (layer "F.Cu") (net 13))
 (via (at 153.25 111.25) (size 0.6) (drill 0.3) (layers "F.Cu" "B.Cu") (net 13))
 (via (at 153.25 92.75) (size 0.6) (drill 0.3) (layers "F.Cu" "B.Cu") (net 13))
 (segment (start 153.25 111.25) (end 153.25 92.75) (width 0.83) (layer "B.Cu") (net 13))
 (segment (start 97.235 98.265) (end 111.275 84.225) (width 0.63) (layer "F.Cu") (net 9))
 (segment (start 97.235 120.5) (end 97.235 98.265) (width 0.63) (layer "F.Cu") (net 9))
 (segment (start 111.275 84.225) (end 111.615 84.225) (width 0.63) (layer "F.Cu") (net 9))
 (segment (start 149.51 83.24) (end 149.51 81.2) (width 0.63) (layer "F.Cu") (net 17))
 (segment (start 149.5 97.5) (end 149.5 89.75) (width 0.63) (layer "F.Cu") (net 17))
 (segment (start 149.51 83.24) (end 149.52 83.25) (width 0.63) (layer "F.Cu") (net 17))
 (segment (start 149.51 81.2) (end 148.31 80) (width 0.63) (layer "F.Cu") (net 17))
 (segment (start 137.015 107.085) (end 139.915 107.085) (width 0.63) (layer "F.Cu") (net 17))
 (segment (start 139.915 107.085) (end 149.5 97.5) (width 0.63) (layer "F.Cu") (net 17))
 (via (at 149.5 89.75) (size 0.6) (drill 0.3) (layers "F.Cu" "B.Cu") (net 17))
 (via (at 149.51 83.24) (size 0.6) (drill 0.3) (layers "F.Cu" "B.Cu") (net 17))
 (segment (start 149.5 83.25) (end 149.5 89.75) (width 0.63) (layer "B.Cu") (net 17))
 (segment (start 149.51 83.24) (end 149.5 83.25) (width 0.63) (layer "B.Cu") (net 17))
 (segment (start 109.5 98) (end 107.5 96) (width 0.83) (layer "F.Cu") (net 18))
 (segment (start 102.5 90.25) (end 102.5 80.54) (width 0.83) (layer "F.Cu") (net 18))
 (segment (start 110.535 119.785) (end 109.5 118.75) (width 0.83) (layer "F.Cu") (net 18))
 (segment (start 111.615 119.785) (end 110.535 119.785) (width 0.83) (layer "F.Cu") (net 18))
 (segment (start 102.5 80.54) (end 102.46 80.5) (width 0.83) (layer "F.Cu") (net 18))
 (segment (start 109.5 109) (end 109.5 98) (width 0.83) (layer "F.Cu") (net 18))
 (via (at 102.5 90) (size 0.6) (drill 0.3) (layers "F.Cu" "B.Cu") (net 18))
 (via (at 109.5 109) (size 0.6) (drill 0.3) (layers "F.Cu" "B.Cu") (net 18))
 (via (at 109.5 118.75) (size 0.6) (drill 0.3) (layers "F.Cu" "B.Cu") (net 18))
 (via (at 107.5 96) (size 0.6) (drill 0.3) (layers "F.Cu" "B.Cu") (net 18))
 (segment (start 102.5 92.25) (end 106.25 96) (width 0.83) (layer "B.Cu") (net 18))
 (segment (start 102.5 90) (end 102.5 92.25) (width 0.83) (layer "B.Cu") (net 18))
 (segment (start 109.5 118.75) (end 109.5 109) (width 0.83) (layer "B.Cu") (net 18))
 (segment (start 106.25 96) (end 107.5 96) (width 0.83) (layer "B.Cu") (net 18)))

